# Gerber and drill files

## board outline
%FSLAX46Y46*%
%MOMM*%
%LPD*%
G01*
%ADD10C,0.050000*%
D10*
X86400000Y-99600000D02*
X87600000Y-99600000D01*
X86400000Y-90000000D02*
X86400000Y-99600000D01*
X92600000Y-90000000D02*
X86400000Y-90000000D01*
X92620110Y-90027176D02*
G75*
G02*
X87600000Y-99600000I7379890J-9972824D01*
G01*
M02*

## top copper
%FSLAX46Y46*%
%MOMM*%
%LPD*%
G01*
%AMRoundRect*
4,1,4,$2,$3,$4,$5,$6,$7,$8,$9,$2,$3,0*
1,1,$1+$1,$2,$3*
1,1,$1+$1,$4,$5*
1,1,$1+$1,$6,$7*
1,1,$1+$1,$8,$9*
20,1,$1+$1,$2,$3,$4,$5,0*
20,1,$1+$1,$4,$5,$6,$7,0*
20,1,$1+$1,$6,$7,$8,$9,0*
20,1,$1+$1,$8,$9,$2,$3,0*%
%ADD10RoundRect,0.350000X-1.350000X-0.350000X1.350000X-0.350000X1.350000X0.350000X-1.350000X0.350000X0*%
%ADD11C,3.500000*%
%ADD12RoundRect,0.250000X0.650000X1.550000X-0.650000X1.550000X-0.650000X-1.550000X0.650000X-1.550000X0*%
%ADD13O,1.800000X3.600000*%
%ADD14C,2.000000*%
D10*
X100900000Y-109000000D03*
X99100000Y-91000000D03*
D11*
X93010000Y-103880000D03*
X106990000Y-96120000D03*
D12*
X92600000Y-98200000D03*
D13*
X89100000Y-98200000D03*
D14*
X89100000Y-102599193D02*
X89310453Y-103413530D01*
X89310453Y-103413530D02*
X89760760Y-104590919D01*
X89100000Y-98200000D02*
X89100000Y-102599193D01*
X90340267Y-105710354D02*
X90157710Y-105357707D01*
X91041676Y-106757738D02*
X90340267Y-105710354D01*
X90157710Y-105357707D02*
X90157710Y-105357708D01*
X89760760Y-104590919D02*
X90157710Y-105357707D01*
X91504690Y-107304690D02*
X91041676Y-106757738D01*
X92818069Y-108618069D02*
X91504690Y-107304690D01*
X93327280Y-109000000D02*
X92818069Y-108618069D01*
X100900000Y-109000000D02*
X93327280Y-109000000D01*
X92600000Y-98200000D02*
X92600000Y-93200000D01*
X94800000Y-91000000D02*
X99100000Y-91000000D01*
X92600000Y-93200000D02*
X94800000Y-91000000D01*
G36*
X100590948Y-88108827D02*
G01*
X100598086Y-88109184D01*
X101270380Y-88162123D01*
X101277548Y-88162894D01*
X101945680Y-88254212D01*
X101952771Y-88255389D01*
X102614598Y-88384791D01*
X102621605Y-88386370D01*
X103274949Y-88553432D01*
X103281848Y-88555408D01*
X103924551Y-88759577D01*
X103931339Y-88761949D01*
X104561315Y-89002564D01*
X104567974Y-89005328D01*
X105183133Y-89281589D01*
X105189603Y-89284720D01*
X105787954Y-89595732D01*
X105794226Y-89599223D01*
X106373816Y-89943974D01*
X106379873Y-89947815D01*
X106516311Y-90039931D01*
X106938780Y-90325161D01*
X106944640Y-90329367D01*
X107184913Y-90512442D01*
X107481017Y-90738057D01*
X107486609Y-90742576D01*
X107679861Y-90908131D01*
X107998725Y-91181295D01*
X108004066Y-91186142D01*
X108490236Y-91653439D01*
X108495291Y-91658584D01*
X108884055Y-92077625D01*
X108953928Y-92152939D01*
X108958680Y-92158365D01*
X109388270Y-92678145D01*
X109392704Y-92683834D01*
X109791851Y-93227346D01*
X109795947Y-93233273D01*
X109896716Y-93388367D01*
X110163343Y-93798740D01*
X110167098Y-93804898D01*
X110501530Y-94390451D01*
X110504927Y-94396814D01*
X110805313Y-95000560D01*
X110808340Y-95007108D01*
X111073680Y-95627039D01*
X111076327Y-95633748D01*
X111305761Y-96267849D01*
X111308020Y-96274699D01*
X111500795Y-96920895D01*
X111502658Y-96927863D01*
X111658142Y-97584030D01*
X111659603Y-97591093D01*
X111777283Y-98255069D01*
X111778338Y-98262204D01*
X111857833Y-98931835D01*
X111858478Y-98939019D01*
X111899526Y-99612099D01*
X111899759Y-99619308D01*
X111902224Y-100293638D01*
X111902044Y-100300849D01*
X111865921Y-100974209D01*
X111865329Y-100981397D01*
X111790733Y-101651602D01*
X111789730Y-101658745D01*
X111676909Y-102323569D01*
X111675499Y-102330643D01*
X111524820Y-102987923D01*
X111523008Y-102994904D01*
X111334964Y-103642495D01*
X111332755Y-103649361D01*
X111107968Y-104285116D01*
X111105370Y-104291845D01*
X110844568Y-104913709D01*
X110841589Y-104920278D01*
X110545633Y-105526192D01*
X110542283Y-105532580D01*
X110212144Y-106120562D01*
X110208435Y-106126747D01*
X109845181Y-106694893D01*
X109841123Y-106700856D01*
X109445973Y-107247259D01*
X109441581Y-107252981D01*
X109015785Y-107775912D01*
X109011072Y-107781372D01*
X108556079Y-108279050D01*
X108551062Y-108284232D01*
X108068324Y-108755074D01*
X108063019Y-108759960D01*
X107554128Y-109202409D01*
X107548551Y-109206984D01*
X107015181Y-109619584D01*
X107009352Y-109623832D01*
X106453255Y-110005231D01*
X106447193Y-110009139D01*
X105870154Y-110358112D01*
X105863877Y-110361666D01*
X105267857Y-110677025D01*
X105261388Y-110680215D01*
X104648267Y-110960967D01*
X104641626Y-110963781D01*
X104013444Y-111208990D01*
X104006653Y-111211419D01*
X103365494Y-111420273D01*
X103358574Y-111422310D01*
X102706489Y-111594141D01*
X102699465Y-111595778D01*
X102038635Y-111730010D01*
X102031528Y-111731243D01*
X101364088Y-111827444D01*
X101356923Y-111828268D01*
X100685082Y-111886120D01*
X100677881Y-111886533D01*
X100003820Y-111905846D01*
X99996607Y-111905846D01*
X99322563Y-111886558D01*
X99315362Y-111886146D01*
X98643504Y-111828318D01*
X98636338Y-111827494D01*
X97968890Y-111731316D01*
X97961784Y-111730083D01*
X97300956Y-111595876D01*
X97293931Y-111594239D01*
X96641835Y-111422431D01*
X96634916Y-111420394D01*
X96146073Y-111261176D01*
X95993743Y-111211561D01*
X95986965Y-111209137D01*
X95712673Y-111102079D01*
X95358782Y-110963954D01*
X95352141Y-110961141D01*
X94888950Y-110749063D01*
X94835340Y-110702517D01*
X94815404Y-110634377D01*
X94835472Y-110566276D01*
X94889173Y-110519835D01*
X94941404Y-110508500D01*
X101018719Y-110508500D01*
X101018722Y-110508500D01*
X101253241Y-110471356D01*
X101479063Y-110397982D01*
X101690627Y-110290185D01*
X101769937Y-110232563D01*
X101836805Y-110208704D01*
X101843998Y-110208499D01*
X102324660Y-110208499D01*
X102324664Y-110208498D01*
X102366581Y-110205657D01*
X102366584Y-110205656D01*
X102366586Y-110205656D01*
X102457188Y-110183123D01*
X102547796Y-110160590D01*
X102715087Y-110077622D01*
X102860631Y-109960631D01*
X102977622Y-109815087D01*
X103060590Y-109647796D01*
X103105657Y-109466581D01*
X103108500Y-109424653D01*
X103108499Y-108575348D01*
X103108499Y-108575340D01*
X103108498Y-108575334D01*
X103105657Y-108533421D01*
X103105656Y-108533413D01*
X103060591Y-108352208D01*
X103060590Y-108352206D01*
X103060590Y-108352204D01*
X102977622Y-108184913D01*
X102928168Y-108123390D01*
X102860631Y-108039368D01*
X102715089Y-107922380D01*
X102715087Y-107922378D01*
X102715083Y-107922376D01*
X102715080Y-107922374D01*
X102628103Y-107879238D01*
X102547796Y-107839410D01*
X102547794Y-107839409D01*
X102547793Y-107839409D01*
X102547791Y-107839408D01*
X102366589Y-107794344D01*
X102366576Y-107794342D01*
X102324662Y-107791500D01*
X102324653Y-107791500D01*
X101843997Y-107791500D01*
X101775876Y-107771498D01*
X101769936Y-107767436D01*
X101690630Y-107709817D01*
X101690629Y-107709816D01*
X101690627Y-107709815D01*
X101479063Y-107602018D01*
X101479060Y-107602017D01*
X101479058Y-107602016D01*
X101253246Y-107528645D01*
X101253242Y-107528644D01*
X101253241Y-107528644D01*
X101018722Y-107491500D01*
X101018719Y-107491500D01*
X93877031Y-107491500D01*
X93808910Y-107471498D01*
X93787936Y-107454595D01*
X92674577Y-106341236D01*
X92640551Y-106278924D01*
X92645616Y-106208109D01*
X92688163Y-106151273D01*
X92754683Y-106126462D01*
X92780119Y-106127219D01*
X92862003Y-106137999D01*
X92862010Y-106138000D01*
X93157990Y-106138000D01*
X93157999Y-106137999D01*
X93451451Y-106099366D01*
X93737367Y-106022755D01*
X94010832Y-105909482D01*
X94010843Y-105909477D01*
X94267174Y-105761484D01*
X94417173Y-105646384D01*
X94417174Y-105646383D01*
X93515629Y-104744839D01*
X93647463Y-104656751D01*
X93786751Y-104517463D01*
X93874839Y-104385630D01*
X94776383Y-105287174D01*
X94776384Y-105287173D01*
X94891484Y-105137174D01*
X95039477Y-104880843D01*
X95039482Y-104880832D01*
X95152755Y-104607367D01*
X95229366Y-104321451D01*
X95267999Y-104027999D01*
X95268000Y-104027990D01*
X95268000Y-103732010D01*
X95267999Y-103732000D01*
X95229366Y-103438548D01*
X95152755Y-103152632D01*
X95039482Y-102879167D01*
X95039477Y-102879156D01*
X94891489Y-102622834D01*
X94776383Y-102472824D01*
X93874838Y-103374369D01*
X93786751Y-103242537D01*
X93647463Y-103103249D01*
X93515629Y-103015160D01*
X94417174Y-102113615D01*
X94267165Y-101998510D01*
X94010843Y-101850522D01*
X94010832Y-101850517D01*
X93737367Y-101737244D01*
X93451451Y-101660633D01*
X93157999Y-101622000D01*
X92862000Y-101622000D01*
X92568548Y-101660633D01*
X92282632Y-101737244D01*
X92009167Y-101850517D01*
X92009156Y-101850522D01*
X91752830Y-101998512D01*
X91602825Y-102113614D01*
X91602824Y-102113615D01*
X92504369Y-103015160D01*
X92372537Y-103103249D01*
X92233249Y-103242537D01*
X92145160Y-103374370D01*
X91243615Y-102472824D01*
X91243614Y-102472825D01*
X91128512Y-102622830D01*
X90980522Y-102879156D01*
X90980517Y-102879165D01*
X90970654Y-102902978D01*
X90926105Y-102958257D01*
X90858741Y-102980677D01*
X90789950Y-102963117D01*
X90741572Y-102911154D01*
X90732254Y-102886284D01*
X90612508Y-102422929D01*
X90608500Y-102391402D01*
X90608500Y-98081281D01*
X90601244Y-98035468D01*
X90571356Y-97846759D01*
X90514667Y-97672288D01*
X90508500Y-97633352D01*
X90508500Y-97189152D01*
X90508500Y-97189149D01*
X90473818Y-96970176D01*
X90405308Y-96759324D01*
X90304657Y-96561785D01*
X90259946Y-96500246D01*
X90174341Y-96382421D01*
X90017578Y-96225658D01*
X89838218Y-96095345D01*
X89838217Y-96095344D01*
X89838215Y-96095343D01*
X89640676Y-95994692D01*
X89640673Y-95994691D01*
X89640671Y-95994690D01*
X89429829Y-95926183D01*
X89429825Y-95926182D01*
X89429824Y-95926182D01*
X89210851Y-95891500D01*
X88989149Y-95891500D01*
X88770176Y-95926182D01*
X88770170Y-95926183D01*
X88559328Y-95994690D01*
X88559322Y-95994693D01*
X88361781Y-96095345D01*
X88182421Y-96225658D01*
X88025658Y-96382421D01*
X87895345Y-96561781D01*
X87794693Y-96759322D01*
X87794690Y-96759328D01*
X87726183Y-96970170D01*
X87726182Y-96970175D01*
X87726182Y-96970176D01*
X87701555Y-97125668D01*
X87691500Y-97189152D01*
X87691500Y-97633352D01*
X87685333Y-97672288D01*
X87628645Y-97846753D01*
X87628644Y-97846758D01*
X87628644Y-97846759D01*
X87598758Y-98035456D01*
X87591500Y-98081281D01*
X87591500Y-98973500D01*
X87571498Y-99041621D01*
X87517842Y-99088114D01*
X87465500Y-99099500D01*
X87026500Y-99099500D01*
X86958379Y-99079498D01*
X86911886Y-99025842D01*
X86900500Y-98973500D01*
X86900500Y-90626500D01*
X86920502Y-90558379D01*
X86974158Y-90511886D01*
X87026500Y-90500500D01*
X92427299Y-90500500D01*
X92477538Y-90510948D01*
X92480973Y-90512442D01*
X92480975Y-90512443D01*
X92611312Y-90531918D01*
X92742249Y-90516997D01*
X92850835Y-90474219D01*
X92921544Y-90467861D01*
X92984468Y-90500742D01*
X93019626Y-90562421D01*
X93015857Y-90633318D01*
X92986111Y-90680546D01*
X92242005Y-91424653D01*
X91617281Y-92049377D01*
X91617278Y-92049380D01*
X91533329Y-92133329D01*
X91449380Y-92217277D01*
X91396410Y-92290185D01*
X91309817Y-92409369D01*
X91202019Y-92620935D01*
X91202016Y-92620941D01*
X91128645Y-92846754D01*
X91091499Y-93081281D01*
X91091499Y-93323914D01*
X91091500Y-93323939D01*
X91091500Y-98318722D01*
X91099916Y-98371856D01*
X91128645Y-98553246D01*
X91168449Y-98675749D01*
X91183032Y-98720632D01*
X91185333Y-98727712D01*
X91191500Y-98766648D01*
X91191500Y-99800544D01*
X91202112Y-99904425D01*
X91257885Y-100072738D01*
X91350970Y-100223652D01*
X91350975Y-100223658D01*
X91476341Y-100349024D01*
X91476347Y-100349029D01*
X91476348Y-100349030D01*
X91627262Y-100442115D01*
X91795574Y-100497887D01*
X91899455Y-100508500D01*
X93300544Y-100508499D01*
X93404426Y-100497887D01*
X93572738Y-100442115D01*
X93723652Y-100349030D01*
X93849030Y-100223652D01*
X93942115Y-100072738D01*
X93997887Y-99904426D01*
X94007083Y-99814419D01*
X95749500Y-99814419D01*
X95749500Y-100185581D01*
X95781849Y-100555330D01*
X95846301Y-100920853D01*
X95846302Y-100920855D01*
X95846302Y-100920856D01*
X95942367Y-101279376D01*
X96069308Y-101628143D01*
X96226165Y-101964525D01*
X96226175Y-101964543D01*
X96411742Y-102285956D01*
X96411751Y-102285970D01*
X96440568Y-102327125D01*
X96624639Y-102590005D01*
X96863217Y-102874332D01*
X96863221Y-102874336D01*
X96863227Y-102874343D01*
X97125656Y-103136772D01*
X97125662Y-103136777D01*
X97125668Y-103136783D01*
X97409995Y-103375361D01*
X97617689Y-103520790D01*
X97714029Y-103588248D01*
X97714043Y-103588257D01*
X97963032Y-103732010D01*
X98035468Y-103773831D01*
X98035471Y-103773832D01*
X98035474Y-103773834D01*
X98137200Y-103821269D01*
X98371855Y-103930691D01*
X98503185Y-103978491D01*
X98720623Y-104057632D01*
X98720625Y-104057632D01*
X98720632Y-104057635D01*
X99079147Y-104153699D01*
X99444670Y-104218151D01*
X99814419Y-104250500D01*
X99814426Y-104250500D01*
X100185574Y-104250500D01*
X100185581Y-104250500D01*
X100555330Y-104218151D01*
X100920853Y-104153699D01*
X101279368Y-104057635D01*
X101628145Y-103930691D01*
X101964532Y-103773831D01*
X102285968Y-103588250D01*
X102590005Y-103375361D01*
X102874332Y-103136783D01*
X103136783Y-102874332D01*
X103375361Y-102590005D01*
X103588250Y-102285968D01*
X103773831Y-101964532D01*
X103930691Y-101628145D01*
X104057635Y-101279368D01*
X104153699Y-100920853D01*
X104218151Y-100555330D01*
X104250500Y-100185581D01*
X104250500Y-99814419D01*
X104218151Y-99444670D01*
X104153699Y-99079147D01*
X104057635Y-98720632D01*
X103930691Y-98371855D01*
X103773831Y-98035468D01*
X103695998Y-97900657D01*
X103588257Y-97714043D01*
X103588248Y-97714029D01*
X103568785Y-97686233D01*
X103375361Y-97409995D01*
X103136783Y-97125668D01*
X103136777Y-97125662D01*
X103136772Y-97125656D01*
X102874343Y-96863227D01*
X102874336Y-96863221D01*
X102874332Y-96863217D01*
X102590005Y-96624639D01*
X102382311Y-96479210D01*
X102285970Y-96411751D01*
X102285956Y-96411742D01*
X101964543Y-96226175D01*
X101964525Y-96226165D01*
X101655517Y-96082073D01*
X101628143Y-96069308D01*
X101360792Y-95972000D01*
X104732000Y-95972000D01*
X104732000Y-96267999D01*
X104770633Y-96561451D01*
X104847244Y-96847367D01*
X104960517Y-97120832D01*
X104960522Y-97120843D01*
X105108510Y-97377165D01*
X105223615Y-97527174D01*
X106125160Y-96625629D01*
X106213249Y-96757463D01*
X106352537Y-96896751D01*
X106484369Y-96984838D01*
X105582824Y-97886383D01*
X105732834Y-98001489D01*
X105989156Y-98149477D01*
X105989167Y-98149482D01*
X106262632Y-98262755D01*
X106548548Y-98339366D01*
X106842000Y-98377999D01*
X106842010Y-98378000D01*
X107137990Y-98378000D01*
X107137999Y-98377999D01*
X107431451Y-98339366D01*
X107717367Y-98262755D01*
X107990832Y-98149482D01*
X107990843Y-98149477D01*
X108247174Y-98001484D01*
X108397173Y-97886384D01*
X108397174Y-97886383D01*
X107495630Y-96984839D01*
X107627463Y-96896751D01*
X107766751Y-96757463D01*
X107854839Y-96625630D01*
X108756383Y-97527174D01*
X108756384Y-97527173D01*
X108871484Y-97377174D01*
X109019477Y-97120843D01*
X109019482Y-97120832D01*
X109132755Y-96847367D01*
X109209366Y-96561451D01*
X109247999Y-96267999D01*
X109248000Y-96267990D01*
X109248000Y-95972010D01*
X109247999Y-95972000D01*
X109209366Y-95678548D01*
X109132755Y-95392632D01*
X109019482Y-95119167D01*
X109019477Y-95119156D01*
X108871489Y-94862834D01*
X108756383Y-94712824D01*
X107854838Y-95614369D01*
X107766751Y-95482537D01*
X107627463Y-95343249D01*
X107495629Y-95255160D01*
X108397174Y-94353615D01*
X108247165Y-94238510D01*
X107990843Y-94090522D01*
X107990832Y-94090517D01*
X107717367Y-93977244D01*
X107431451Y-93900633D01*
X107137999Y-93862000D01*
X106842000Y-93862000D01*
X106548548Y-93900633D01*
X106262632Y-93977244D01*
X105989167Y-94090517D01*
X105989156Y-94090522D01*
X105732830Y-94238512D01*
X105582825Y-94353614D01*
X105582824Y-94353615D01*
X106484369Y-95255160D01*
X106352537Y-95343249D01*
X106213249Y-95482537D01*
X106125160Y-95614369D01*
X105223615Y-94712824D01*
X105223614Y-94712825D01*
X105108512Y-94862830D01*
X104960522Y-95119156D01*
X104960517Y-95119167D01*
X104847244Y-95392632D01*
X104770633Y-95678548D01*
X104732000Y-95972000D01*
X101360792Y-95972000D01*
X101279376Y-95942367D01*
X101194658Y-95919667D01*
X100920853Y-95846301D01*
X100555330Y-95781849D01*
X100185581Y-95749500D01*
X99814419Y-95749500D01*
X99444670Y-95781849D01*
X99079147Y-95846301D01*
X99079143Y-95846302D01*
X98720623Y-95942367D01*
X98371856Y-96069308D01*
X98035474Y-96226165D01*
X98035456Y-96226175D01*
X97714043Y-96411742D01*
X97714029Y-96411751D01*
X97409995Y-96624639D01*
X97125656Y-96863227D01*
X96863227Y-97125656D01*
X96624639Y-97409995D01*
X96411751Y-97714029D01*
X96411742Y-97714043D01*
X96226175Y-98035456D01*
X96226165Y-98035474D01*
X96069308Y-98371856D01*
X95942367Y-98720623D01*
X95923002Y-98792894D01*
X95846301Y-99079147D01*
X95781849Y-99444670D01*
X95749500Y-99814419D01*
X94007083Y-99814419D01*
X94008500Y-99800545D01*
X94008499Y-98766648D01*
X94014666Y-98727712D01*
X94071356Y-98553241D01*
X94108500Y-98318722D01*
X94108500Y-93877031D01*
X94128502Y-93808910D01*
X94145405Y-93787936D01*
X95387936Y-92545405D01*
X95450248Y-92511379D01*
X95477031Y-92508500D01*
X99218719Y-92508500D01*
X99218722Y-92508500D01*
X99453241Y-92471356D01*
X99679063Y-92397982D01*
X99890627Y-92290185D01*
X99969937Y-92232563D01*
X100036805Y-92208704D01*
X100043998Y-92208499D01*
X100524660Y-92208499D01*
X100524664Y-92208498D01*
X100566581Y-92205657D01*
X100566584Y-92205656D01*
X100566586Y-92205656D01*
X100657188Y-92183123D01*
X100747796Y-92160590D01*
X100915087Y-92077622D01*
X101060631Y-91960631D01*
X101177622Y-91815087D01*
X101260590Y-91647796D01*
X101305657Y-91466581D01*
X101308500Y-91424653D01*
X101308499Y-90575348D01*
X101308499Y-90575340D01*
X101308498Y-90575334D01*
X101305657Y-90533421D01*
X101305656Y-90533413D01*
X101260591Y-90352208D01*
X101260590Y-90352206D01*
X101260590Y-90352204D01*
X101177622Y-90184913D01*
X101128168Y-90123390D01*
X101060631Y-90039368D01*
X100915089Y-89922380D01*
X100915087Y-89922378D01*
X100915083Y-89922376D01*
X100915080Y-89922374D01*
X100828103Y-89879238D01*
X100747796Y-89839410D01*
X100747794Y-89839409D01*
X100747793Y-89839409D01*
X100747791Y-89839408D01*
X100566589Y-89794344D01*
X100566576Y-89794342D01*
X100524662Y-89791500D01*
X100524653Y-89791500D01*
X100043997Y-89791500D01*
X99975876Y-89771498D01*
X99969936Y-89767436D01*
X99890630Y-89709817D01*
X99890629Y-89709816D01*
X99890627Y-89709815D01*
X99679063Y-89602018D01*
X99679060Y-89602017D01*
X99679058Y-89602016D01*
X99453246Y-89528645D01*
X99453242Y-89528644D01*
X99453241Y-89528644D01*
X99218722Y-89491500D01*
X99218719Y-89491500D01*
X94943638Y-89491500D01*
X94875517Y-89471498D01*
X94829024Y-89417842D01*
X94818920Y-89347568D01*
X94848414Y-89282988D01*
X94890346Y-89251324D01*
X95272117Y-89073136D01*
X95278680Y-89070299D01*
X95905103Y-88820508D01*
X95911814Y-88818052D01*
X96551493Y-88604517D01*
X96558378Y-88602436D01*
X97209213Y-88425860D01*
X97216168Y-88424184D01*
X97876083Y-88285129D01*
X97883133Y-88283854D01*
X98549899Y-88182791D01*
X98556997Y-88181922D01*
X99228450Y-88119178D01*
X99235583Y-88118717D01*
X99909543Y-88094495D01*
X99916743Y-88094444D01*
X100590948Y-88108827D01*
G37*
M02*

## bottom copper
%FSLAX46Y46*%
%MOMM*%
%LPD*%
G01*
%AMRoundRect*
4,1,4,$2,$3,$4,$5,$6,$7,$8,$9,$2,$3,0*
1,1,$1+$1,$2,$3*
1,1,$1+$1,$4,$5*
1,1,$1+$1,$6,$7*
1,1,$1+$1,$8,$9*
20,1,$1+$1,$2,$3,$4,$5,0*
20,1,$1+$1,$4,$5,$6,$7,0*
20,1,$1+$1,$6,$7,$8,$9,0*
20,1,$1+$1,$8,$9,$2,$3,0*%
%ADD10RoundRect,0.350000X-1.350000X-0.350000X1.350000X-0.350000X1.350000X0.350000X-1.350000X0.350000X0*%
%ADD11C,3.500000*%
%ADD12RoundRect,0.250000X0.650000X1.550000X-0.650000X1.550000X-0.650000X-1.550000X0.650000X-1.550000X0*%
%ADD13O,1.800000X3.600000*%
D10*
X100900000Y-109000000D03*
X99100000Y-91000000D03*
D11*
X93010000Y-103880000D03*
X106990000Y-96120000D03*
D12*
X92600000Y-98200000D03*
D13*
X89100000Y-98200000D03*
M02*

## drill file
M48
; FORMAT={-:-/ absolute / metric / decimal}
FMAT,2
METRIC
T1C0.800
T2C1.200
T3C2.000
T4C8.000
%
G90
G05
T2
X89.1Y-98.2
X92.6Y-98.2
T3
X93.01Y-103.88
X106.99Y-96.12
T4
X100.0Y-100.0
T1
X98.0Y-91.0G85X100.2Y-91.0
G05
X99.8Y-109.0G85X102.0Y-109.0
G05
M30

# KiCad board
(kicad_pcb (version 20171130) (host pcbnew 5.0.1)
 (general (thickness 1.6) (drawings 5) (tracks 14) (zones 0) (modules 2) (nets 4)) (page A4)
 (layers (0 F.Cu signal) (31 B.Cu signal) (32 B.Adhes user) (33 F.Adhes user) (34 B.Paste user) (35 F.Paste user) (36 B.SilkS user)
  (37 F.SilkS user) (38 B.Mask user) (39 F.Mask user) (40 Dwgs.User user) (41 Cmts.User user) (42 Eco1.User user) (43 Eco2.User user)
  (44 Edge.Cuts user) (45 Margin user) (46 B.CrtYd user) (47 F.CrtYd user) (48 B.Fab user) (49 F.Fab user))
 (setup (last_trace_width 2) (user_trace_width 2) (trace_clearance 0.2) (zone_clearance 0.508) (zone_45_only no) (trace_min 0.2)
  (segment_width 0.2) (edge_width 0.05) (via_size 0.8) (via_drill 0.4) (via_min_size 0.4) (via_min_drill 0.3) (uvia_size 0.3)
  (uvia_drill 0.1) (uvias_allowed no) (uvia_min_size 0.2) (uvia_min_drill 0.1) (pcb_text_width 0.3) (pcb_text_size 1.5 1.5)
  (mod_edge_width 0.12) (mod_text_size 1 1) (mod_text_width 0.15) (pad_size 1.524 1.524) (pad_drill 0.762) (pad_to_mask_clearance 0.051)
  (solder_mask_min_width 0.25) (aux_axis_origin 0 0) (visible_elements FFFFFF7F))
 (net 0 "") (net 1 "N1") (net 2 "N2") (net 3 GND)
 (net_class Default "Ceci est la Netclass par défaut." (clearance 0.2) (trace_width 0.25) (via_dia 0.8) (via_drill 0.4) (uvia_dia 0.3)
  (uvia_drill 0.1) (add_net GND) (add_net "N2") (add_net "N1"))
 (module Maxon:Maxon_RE (layer F.Cu) (at 100 100 270)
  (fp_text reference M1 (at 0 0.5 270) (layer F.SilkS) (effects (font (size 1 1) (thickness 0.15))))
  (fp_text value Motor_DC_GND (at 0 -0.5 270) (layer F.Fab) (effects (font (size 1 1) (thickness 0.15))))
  (pad 1 thru_hole roundrect (at 9 -0.9) (size 3.4 1.4) (drill oval 3 0.8) (layers *.Cu *.Mask) (roundrect_rratio 0.25) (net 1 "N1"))
  (pad 2 thru_hole roundrect (at -9 0.9) (size 3.4 1.4) (drill oval 3 0.8) (layers *.Cu *.Mask) (roundrect_rratio 0.25) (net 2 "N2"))
  (pad 3 thru_hole circle (at 3.88 6.99 270) (size 3.5 3.5) (drill 2) (layers *.Cu *.Mask) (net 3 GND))
  (pad 3 thru_hole circle (at -3.88 -6.99 270) (size 3.5 3.5) (drill 2) (layers *.Cu *.Mask) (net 3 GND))
  (pad "" np_thru_hole circle (at 0 0 270) (size 8 8) (drill 8) (layers *.Cu *.Mask)))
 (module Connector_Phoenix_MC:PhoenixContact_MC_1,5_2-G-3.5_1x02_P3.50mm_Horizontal (layer F.Cu) (at 92.6 98.2 180)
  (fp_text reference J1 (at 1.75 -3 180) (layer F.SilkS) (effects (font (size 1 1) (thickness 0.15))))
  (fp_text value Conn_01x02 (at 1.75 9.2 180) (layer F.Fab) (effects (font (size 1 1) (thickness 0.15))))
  (pad 1 thru_hole roundrect (at 0 0 180) (size 1.8 3.6) (drill 1.2) (layers *.Cu *.Mask) (roundrect_rratio 0.138889) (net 2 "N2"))
  (pad 2 thru_hole oval (at 3.5 0 180) (size 1.8 3.6) (drill 1.2) (layers *.Cu *.Mask) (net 1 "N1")))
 (gr_line (start 86.4 99.6) (end 87.6 99.6) (layer Edge.Cuts) (width 0.05))
 (gr_line (start 86.4 90) (end 86.4 99.6) (layer Edge.Cuts) (width 0.05))
 (gr_line (start 92.6 90) (end 86.4 90) (layer Edge.Cuts) (width 0.05))
 (gr_arc (start 100 100) (end 87.6 99.6) (angle -308.3490523) (layer Edge.Cuts) (width 0.05))
 (segment (start 89.1 102.599193) (end 89.310453 103.41353) (width 2) (layer F.Cu) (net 1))
 (segment (start 89.310453 103.41353) (end 89.76076 104.590919) (width 2) (layer F.Cu) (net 1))
 (segment (start 89.1 98.2) (end 89.1 102.599193) (width 2) (layer F.Cu) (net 1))
 (segment (start 90.340267 105.710354) (end 90.15771 105.357707) (width 2) (layer F.Cu) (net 1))
 (segment (start 91.041676 106.757738) (end 90.340267 105.710354) (width 2) (layer F.Cu) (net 1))
 (segment (start 90.15771 105.357707) (end 90.15771 105.357708) (width 2) (layer F.Cu) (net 1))
 (segment (start 89.76076 104.590919) (end 90.15771 105.357707) (width 2) (layer F.Cu) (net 1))
 (segment (start 91.50469 107.30469) (end 91.041676 106.757738) (width 2) (layer F.Cu) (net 1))
 (segment (start 92.818069 108.618069) (end 91.50469 107.30469) (width 2) (layer F.Cu) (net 1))
 (segment (start 93.32728 109) (end 92.818069 108.618069) (width 2) (layer F.Cu) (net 1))
 (segment (start 100.9 109) (end 93.32728 109) (width 2) (layer F.Cu) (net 1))
 (segment (start 92.6 98.2) (end 92.6 93.2) (width 2) (layer F.Cu) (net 2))
 (segment (start 94.8 91) (end 99.1 91) (width 2) (layer F.Cu) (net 2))
 (segment (start 92.6 93.2) (end 94.8 91) (width 2) (layer F.Cu) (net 2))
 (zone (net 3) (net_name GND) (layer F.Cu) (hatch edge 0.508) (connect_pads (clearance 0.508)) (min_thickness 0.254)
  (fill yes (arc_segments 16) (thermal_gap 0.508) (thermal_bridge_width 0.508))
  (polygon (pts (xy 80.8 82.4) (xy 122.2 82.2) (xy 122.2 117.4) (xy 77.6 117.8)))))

